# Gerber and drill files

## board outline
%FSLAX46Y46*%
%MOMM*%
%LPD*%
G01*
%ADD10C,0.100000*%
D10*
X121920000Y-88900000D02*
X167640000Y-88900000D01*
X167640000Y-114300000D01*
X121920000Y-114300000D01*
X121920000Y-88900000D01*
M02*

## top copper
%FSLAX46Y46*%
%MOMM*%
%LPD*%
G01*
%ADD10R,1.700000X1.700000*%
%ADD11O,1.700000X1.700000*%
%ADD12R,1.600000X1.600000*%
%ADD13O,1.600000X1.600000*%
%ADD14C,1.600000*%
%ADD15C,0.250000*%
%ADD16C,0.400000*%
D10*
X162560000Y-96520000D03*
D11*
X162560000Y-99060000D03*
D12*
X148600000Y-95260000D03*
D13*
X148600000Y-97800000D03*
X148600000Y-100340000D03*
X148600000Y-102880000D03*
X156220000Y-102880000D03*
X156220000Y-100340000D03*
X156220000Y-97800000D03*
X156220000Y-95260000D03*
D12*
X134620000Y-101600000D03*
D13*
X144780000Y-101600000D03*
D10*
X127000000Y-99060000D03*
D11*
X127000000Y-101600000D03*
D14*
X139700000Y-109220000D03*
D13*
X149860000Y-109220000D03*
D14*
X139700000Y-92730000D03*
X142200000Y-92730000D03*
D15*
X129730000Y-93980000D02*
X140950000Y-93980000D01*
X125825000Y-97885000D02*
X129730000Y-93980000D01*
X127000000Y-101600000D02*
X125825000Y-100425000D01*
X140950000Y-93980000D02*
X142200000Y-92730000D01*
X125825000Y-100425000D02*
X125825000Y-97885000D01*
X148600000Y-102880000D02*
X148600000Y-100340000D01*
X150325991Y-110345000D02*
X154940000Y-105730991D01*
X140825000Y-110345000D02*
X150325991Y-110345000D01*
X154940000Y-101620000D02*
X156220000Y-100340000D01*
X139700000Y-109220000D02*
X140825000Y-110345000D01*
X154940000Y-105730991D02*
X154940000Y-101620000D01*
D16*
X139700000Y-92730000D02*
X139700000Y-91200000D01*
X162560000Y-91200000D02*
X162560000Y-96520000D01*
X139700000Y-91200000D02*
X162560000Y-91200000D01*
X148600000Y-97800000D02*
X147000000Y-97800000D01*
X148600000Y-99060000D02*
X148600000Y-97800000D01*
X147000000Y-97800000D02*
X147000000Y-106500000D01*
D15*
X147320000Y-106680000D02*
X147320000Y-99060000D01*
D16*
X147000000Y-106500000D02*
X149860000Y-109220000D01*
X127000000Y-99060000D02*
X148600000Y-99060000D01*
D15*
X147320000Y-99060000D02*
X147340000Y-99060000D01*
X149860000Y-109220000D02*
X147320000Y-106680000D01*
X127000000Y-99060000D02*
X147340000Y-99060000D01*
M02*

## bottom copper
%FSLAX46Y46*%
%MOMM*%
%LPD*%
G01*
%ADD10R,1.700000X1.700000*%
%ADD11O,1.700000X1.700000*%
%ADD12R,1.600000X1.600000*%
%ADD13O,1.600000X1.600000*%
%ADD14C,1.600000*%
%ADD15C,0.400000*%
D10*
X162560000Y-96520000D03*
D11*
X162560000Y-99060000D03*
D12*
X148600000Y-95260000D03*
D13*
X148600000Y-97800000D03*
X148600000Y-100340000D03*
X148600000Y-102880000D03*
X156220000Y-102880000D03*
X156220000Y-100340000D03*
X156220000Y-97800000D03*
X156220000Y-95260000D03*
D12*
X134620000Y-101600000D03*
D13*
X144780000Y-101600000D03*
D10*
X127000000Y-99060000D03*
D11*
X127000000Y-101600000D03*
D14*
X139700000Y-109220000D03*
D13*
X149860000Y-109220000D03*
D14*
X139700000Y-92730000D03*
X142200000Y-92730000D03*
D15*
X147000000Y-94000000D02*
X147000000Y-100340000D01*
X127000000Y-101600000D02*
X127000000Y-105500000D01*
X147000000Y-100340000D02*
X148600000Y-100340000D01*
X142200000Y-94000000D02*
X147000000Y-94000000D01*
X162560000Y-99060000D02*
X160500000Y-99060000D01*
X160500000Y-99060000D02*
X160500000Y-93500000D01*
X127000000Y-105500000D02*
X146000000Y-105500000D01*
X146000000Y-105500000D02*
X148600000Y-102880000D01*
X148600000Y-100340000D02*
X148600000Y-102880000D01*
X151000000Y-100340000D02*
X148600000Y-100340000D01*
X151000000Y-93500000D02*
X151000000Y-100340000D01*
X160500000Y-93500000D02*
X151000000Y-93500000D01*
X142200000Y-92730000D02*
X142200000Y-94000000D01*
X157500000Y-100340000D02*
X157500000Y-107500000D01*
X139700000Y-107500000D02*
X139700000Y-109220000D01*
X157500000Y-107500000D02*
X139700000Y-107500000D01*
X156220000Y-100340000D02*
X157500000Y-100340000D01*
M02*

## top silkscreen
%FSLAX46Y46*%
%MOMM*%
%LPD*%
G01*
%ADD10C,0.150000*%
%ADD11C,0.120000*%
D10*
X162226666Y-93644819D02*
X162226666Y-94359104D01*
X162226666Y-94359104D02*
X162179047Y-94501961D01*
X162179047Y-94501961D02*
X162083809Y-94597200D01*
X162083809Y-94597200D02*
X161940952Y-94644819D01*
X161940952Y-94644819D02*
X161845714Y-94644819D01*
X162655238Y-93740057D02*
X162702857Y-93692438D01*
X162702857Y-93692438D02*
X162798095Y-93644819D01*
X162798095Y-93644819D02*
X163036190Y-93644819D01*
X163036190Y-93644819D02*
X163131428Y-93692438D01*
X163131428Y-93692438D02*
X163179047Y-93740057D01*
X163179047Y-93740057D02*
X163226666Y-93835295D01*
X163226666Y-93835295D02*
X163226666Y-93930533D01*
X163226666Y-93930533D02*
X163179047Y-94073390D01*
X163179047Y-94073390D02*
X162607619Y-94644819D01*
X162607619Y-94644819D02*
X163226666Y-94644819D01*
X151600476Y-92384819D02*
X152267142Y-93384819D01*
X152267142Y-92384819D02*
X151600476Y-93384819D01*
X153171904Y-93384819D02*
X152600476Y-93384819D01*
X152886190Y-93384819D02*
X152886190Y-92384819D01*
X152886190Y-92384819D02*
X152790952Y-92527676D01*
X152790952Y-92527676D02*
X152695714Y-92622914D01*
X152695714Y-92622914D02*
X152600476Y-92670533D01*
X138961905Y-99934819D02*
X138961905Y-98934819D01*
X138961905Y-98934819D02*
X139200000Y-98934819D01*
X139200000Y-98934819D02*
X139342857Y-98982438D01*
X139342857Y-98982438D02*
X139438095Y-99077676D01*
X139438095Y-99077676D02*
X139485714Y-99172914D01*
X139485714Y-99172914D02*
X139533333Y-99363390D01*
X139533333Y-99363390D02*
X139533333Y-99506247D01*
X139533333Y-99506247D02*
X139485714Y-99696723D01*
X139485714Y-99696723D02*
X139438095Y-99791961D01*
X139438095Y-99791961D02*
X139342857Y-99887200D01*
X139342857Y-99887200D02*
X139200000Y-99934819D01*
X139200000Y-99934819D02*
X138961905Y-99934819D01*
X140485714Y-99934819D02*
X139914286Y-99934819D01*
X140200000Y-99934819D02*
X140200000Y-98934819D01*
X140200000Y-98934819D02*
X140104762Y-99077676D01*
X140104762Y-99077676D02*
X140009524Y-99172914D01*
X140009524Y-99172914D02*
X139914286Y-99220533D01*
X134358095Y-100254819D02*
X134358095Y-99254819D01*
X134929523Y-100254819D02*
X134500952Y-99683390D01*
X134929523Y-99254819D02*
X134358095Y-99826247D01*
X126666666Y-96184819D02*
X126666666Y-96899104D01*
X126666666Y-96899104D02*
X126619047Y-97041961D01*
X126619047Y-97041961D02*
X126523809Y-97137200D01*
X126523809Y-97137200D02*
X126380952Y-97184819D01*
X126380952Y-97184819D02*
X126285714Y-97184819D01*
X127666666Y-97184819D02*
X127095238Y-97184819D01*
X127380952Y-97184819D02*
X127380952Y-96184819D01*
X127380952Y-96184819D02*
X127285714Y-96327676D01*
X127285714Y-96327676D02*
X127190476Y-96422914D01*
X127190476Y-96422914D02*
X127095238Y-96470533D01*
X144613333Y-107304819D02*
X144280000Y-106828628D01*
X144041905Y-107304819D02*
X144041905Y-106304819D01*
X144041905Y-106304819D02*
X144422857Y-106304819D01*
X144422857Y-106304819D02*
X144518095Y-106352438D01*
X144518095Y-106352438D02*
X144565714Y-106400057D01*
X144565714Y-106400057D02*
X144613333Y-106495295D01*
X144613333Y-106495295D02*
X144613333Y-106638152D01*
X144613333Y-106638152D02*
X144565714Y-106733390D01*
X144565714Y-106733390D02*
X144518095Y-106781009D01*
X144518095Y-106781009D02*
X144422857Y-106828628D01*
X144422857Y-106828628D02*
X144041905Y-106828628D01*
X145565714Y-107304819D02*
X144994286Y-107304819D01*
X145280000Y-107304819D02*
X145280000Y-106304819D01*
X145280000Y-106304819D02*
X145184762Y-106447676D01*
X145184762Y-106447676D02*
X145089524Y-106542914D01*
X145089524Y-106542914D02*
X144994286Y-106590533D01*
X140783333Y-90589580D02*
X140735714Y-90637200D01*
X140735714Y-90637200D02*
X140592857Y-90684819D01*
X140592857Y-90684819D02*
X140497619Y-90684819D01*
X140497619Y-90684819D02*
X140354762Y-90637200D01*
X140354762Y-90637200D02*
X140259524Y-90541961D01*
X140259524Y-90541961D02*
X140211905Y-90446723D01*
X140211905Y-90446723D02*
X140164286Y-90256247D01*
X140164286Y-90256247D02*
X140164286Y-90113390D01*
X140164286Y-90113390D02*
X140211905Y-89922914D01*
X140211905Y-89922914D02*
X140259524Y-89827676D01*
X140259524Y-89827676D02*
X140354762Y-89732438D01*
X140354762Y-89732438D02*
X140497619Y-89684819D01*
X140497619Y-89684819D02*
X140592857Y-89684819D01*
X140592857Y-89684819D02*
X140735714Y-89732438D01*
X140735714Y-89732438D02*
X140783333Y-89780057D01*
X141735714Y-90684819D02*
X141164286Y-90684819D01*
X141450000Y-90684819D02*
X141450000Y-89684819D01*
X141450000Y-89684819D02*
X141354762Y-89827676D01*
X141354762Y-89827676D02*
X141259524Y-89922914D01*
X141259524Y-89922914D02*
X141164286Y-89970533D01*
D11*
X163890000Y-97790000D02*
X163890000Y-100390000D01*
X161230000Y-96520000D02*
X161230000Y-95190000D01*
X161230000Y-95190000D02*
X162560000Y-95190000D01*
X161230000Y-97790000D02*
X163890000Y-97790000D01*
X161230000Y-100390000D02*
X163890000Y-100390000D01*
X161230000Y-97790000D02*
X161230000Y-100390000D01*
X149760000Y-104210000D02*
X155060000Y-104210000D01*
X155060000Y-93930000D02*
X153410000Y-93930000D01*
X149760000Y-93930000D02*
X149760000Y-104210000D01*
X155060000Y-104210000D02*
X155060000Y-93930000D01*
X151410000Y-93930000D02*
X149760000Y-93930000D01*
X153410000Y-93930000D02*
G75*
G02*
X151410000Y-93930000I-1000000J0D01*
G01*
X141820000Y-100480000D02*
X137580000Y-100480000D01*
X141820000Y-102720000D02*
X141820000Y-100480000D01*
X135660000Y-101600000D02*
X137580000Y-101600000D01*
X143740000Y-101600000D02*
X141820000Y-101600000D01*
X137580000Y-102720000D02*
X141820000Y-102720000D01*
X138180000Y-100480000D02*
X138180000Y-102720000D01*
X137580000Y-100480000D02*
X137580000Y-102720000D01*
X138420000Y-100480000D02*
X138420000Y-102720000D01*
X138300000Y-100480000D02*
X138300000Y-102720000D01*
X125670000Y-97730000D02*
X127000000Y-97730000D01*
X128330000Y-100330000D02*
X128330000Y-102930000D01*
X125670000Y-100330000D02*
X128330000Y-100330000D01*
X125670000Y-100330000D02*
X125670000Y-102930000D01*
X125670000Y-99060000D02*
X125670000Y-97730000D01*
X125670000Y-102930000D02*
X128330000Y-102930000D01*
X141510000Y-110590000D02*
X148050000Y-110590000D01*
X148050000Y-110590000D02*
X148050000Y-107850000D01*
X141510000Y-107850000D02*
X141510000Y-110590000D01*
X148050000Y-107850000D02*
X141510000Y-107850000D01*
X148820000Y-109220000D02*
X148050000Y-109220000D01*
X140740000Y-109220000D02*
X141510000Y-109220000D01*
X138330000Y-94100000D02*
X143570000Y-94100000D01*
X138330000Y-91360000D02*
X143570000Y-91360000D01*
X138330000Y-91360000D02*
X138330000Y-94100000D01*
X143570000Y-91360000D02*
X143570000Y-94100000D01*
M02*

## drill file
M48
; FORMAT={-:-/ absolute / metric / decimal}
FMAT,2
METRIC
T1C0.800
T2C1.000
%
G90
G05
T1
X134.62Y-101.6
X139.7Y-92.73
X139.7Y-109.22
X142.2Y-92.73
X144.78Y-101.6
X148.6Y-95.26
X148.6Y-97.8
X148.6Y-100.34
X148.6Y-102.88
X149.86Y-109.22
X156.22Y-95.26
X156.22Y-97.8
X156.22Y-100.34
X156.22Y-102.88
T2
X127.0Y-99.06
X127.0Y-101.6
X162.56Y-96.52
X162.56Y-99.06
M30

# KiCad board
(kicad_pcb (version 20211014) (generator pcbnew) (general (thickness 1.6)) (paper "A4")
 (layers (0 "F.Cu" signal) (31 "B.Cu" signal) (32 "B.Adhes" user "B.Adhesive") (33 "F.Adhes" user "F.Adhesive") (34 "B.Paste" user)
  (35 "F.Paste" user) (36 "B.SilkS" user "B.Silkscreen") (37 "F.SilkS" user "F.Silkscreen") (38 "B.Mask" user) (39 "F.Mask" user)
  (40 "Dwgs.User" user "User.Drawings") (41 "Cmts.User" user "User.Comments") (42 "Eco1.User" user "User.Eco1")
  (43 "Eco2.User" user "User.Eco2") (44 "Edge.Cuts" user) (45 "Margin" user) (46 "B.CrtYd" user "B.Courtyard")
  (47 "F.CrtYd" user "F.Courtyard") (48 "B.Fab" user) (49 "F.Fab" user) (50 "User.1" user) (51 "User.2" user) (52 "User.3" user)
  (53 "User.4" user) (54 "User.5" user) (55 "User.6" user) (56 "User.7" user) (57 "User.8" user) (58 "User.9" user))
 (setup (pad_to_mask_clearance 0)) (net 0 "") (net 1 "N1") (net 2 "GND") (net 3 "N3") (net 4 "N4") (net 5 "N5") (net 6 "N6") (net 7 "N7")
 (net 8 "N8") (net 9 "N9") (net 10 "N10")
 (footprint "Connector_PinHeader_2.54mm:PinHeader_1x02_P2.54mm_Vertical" (layer "F.Cu") (at 162.56 96.52)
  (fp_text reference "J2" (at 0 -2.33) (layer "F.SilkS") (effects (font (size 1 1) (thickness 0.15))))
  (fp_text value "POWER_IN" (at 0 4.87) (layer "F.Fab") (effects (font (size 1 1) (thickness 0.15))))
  (fp_line (start 1.33 1.27) (end 1.33 3.87) (layer "F.SilkS") (width 0.12))
  (fp_line (start -1.33 0) (end -1.33 -1.33) (layer "F.SilkS") (width 0.12))
  (fp_line (start -1.33 -1.33) (end 0 -1.33) (layer "F.SilkS") (width 0.12))
  (fp_line (start -1.33 1.27) (end 1.33 1.27) (layer "F.SilkS") (width 0.12))
  (fp_line (start -1.33 3.87) (end 1.33 3.87) (layer "F.SilkS") (width 0.12))
  (fp_line (start -1.33 1.27) (end -1.33 3.87) (layer "F.SilkS") (width 0.12))
  (pad "1" thru_hole rect (at 0 0) (size 1.7 1.7) (drill 1) (layers *.Cu *.Mask) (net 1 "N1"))
  (pad "2" thru_hole oval (at 0 2.54) (size 1.7 1.7) (drill 1) (layers *.Cu *.Mask) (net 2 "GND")))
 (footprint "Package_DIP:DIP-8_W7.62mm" (layer "F.Cu") (at 148.6 95.26)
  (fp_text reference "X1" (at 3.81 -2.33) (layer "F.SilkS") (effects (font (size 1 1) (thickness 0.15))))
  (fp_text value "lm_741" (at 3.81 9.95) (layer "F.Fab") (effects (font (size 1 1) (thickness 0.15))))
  (fp_line (start 1.16 8.95) (end 6.46 8.95) (layer "F.SilkS") (width 0.12))
  (fp_line (start 6.46 -1.33) (end 4.81 -1.33) (layer "F.SilkS") (width 0.12))
  (fp_line (start 1.16 -1.33) (end 1.16 8.95) (layer "F.SilkS") (width 0.12))
  (fp_line (start 6.46 8.95) (end 6.46 -1.33) (layer "F.SilkS") (width 0.12))
  (fp_line (start 2.81 -1.33) (end 1.16 -1.33) (layer "F.SilkS") (width 0.12))
  (fp_arc (start 4.81 -1.33) (mid 3.81 -0.33) (end 2.81 -1.33) (layer "F.SilkS") (width 0.12))
  (pad "1" thru_hole rect (at 0 0) (size 1.6 1.6) (drill 0.8) (layers *.Cu *.Mask) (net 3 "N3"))
  (pad "2" thru_hole oval (at 0 2.54) (size 1.6 1.6) (drill 0.8) (layers *.Cu *.Mask) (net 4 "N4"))
  (pad "3" thru_hole oval (at 0 5.08) (size 1.6 1.6) (drill 0.8) (layers *.Cu *.Mask) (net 2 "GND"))
  (pad "4" thru_hole oval (at 0 7.62) (size 1.6 1.6) (drill 0.8) (layers *.Cu *.Mask) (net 2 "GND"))
  (pad "5" thru_hole oval (at 7.62 7.62) (size 1.6 1.6) (drill 0.8) (layers *.Cu *.Mask) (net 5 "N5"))
  (pad "6" thru_hole oval (at 7.62 5.08) (size 1.6 1.6) (drill 0.8) (layers *.Cu *.Mask) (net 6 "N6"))
  (pad "7" thru_hole oval (at 7.62 2.54) (size 1.6 1.6) (drill 0.8) (layers *.Cu *.Mask) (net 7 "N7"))
  (pad "8" thru_hole oval (at 7.62 0) (size 1.6 1.6) (drill 0.8) (layers *.Cu *.Mask) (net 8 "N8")))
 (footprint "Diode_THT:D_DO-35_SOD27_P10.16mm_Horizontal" (layer "F.Cu") (at 134.62 101.6)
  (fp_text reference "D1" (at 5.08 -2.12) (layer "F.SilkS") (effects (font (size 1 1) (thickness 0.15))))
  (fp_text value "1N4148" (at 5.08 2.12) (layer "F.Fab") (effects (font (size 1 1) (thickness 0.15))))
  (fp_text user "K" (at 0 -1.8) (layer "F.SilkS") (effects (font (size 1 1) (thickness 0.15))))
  (fp_line (start 7.2 -1.12) (end 2.96 -1.12) (layer "F.SilkS") (width 0.12))
  (fp_line (start 7.2 1.12) (end 7.2 -1.12) (layer "F.SilkS") (width 0.12))
  (fp_line (start 1.04 0) (end 2.96 0) (layer "F.SilkS") (width 0.12))
  (fp_line (start 9.12 0) (end 7.2 0) (layer "F.SilkS") (width 0.12))
  (fp_line (start 2.96 1.12) (end 7.2 1.12) (layer "F.SilkS") (width 0.12))
  (fp_line (start 3.56 -1.12) (end 3.56 1.12) (layer "F.SilkS") (width 0.12))
  (fp_line (start 2.96 -1.12) (end 2.96 1.12) (layer "F.SilkS") (width 0.12))
  (fp_line (start 3.8 -1.12) (end 3.8 1.12) (layer "F.SilkS") (width 0.12))
  (fp_line (start 3.68 -1.12) (end 3.68 1.12) (layer "F.SilkS") (width 0.12))
  (pad "1" thru_hole rect (at 0 0) (size 1.6 1.6) (drill 0.8) (layers *.Cu *.Mask) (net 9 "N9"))
  (pad "2" thru_hole oval (at 10.16 0) (size 1.6 1.6) (drill 0.8) (layers *.Cu *.Mask) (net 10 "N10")))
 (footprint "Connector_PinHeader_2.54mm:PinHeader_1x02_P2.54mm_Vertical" (layer "F.Cu") (at 127 99.06)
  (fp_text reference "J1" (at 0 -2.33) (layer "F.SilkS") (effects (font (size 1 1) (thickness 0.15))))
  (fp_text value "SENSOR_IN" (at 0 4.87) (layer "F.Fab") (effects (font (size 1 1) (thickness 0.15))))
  (fp_line (start -1.33 -1.33) (end 0 -1.33) (layer "F.SilkS") (width 0.12))
  (fp_line (start 1.33 1.27) (end 1.33 3.87) (layer "F.SilkS") (width 0.12))
  (fp_line (start -1.33 1.27) (end 1.33 1.27) (layer "F.SilkS") (width 0.12))
  (fp_line (start -1.33 1.27) (end -1.33 3.87) (layer "F.SilkS") (width 0.12))
  (fp_line (start -1.33 0) (end -1.33 -1.33) (layer "F.SilkS") (width 0.12))
  (fp_line (start -1.33 3.87) (end 1.33 3.87) (layer "F.SilkS") (width 0.12))
  (pad "1" thru_hole rect (at 0 0) (size 1.7 1.7) (drill 1) (layers *.Cu *.Mask) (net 4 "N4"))
  (pad "2" thru_hole oval (at 0 2.54) (size 1.7 1.7) (drill 1) (layers *.Cu *.Mask) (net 2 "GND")))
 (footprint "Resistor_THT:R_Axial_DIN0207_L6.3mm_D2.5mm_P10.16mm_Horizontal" (layer "F.Cu") (at 139.7 109.22)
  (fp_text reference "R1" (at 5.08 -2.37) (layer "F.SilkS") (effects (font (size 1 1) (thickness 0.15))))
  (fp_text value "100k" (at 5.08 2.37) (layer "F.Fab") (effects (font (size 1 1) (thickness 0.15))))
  (fp_line (start 1.81 1.37) (end 8.35 1.37) (layer "F.SilkS") (width 0.12))
  (fp_line (start 8.35 1.37) (end 8.35 -1.37) (layer "F.SilkS") (width 0.12))
  (fp_line (start 1.81 -1.37) (end 1.81 1.37) (layer "F.SilkS") (width 0.12))
  (fp_line (start 8.35 -1.37) (end 1.81 -1.37) (layer "F.SilkS") (width 0.12))
  (fp_line (start 9.12 0) (end 8.35 0) (layer "F.SilkS") (width 0.12))
  (fp_line (start 1.04 0) (end 1.81 0) (layer "F.SilkS") (width 0.12))
  (pad "1" thru_hole circle (at 0 0) (size 1.6 1.6) (drill 0.8) (layers *.Cu *.Mask) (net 6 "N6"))
  (pad "2" thru_hole oval (at 10.16 0) (size 1.6 1.6) (drill 0.8) (layers *.Cu *.Mask) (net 4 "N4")))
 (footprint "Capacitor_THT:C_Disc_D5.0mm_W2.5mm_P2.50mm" (layer "F.Cu") (at 139.7 92.73)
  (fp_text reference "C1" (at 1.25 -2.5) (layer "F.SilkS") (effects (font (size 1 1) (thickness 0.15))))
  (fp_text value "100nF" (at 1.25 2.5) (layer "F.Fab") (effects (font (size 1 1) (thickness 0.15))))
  (fp_line (start -1.37 1.37) (end 3.87 1.37) (layer "F.SilkS") (width 0.12))
  (fp_line (start -1.37 -1.37) (end 3.87 -1.37) (layer "F.SilkS") (width 0.12))
  (fp_line (start -1.37 -1.37) (end -1.37 1.37) (layer "F.SilkS") (width 0.12))
  (fp_line (start 3.87 -1.37) (end 3.87 1.37) (layer "F.SilkS") (width 0.12))
  (pad "1" thru_hole circle (at 0 0) (size 1.6 1.6) (drill 0.8) (layers *.Cu *.Mask) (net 1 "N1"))
  (pad "2" thru_hole circle (at 2.5 0) (size 1.6 1.6) (drill 0.8) (layers *.Cu *.Mask) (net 2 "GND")))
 (gr_rect (start 167.64 114.3) (end 121.92 88.9) (layer "Edge.Cuts") (width 0.1) (fill none))
 (gr_rect (start 147.32 93.98) (end 147.32 93.98) (layer "Edge.Cuts") (width 0.05) (fill none))
 (segment (start 129.73 93.98) (end 140.95 93.98) (width 0.25) (layer "F.Cu") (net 2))
 (segment (start 125.825 97.885) (end 129.73 93.98) (width 0.25) (layer "F.Cu") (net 2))
 (segment (start 127 101.6) (end 125.825 100.425) (width 0.25) (layer "F.Cu") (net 2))
 (segment (start 140.95 93.98) (end 142.2 92.73) (width 0.25) (layer "F.Cu") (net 2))
 (segment (start 125.825 100.425) (end 125.825 97.885) (width 0.25) (layer "F.Cu") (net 2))
 (segment (start 148.6 102.88) (end 148.6 100.34) (width 0.25) (layer "F.Cu") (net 2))
 (segment (start 147 94) (end 147 100.34) (width 0.4) (layer "B.Cu") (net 2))
 (segment (start 127 101.6) (end 127 105.5) (width 0.4) (layer "B.Cu") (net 2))
 (segment (start 147 100.34) (end 148.6 100.34) (width 0.4) (layer "B.Cu") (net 2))
 (segment (start 142.2 94) (end 147 94) (width 0.4) (layer "B.Cu") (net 2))
 (segment (start 162.56 99.06) (end 160.5 99.06) (width 0.4) (layer "B.Cu") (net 2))
 (segment (start 160.5 99.06) (end 160.5 93.5) (width 0.4) (layer "B.Cu") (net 2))
 (segment (start 127 105.5) (end 146 105.5) (width 0.4) (layer "B.Cu") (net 2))
 (segment (start 146 105.5) (end 148.6 102.88) (width 0.4) (layer "B.Cu") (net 2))
 (segment (start 148.6 100.34) (end 148.6 102.88) (width 0.4) (layer "B.Cu") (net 2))
 (segment (start 151 100.34) (end 148.6 100.34) (width 0.4) (layer "B.Cu") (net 2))
 (segment (start 151 93.5) (end 151 100.34) (width 0.4) (layer "B.Cu") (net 2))
 (segment (start 160.5 93.5) (end 151 93.5) (width 0.4) (layer "B.Cu") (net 2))
 (segment (start 142.2 92.73) (end 142.2 94) (width 0.4) (layer "B.Cu") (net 2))
 (segment (start 150.325991 110.345) (end 154.94 105.730991) (width 0.25) (layer "F.Cu") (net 6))
 (segment (start 140.825 110.345) (end 150.325991 110.345) (width 0.25) (layer "F.Cu") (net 6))
 (segment (start 154.94 101.62) (end 156.22 100.34) (width 0.25) (layer "F.Cu") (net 6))
 (segment (start 139.7 109.22) (end 140.825 110.345) (width 0.25) (layer "F.Cu") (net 6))
 (segment (start 154.94 105.730991) (end 154.94 101.62) (width 0.25) (layer "F.Cu") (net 6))
 (segment (start 157.5 100.34) (end 157.5 107.5) (width 0.4) (layer "B.Cu") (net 6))
 (segment (start 139.7 107.5) (end 139.7 109.22) (width 0.4) (layer "B.Cu") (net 6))
 (segment (start 157.5 107.5) (end 139.7 107.5) (width 0.4) (layer "B.Cu") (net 6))
 (segment (start 156.22 100.34) (end 157.5 100.34) (width 0.4) (layer "B.Cu") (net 6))
 (segment (start 139.7 92.73) (end 139.7 91.2) (width 0.4) (layer "F.Cu") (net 1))
 (segment (start 162.56 91.2) (end 162.56 96.52) (width 0.4) (layer "F.Cu") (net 1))
 (segment (start 139.7 91.2) (end 162.56 91.2) (width 0.4) (layer "F.Cu") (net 1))
 (segment (start 148.6 97.8) (end 147 97.8) (width 0.4) (layer "F.Cu") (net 4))
 (segment (start 148.6 99.06) (end 148.6 97.8) (width 0.4) (layer "F.Cu") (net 4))
 (segment (start 147 97.8) (end 147 106.5) (width 0.4) (layer "F.Cu") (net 4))
 (segment (start 147.32 106.68) (end 147.32 99.06) (width 0.25) (layer "F.Cu") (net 4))
 (segment (start 147 106.5) (end 149.86 109.22) (width 0.4) (layer "F.Cu") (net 4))
 (segment (start 127 99.06) (end 148.6 99.06) (width 0.4) (layer "F.Cu") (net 4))
 (segment (start 147.32 99.06) (end 147.34 99.06) (width 0.25) (layer "F.Cu") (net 4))
 (segment (start 149.86 109.22) (end 147.32 106.68) (width 0.25) (layer "F.Cu") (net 4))
 (segment (start 127 99.06) (end 147.34 99.06) (width 0.25) (layer "F.Cu") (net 4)))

